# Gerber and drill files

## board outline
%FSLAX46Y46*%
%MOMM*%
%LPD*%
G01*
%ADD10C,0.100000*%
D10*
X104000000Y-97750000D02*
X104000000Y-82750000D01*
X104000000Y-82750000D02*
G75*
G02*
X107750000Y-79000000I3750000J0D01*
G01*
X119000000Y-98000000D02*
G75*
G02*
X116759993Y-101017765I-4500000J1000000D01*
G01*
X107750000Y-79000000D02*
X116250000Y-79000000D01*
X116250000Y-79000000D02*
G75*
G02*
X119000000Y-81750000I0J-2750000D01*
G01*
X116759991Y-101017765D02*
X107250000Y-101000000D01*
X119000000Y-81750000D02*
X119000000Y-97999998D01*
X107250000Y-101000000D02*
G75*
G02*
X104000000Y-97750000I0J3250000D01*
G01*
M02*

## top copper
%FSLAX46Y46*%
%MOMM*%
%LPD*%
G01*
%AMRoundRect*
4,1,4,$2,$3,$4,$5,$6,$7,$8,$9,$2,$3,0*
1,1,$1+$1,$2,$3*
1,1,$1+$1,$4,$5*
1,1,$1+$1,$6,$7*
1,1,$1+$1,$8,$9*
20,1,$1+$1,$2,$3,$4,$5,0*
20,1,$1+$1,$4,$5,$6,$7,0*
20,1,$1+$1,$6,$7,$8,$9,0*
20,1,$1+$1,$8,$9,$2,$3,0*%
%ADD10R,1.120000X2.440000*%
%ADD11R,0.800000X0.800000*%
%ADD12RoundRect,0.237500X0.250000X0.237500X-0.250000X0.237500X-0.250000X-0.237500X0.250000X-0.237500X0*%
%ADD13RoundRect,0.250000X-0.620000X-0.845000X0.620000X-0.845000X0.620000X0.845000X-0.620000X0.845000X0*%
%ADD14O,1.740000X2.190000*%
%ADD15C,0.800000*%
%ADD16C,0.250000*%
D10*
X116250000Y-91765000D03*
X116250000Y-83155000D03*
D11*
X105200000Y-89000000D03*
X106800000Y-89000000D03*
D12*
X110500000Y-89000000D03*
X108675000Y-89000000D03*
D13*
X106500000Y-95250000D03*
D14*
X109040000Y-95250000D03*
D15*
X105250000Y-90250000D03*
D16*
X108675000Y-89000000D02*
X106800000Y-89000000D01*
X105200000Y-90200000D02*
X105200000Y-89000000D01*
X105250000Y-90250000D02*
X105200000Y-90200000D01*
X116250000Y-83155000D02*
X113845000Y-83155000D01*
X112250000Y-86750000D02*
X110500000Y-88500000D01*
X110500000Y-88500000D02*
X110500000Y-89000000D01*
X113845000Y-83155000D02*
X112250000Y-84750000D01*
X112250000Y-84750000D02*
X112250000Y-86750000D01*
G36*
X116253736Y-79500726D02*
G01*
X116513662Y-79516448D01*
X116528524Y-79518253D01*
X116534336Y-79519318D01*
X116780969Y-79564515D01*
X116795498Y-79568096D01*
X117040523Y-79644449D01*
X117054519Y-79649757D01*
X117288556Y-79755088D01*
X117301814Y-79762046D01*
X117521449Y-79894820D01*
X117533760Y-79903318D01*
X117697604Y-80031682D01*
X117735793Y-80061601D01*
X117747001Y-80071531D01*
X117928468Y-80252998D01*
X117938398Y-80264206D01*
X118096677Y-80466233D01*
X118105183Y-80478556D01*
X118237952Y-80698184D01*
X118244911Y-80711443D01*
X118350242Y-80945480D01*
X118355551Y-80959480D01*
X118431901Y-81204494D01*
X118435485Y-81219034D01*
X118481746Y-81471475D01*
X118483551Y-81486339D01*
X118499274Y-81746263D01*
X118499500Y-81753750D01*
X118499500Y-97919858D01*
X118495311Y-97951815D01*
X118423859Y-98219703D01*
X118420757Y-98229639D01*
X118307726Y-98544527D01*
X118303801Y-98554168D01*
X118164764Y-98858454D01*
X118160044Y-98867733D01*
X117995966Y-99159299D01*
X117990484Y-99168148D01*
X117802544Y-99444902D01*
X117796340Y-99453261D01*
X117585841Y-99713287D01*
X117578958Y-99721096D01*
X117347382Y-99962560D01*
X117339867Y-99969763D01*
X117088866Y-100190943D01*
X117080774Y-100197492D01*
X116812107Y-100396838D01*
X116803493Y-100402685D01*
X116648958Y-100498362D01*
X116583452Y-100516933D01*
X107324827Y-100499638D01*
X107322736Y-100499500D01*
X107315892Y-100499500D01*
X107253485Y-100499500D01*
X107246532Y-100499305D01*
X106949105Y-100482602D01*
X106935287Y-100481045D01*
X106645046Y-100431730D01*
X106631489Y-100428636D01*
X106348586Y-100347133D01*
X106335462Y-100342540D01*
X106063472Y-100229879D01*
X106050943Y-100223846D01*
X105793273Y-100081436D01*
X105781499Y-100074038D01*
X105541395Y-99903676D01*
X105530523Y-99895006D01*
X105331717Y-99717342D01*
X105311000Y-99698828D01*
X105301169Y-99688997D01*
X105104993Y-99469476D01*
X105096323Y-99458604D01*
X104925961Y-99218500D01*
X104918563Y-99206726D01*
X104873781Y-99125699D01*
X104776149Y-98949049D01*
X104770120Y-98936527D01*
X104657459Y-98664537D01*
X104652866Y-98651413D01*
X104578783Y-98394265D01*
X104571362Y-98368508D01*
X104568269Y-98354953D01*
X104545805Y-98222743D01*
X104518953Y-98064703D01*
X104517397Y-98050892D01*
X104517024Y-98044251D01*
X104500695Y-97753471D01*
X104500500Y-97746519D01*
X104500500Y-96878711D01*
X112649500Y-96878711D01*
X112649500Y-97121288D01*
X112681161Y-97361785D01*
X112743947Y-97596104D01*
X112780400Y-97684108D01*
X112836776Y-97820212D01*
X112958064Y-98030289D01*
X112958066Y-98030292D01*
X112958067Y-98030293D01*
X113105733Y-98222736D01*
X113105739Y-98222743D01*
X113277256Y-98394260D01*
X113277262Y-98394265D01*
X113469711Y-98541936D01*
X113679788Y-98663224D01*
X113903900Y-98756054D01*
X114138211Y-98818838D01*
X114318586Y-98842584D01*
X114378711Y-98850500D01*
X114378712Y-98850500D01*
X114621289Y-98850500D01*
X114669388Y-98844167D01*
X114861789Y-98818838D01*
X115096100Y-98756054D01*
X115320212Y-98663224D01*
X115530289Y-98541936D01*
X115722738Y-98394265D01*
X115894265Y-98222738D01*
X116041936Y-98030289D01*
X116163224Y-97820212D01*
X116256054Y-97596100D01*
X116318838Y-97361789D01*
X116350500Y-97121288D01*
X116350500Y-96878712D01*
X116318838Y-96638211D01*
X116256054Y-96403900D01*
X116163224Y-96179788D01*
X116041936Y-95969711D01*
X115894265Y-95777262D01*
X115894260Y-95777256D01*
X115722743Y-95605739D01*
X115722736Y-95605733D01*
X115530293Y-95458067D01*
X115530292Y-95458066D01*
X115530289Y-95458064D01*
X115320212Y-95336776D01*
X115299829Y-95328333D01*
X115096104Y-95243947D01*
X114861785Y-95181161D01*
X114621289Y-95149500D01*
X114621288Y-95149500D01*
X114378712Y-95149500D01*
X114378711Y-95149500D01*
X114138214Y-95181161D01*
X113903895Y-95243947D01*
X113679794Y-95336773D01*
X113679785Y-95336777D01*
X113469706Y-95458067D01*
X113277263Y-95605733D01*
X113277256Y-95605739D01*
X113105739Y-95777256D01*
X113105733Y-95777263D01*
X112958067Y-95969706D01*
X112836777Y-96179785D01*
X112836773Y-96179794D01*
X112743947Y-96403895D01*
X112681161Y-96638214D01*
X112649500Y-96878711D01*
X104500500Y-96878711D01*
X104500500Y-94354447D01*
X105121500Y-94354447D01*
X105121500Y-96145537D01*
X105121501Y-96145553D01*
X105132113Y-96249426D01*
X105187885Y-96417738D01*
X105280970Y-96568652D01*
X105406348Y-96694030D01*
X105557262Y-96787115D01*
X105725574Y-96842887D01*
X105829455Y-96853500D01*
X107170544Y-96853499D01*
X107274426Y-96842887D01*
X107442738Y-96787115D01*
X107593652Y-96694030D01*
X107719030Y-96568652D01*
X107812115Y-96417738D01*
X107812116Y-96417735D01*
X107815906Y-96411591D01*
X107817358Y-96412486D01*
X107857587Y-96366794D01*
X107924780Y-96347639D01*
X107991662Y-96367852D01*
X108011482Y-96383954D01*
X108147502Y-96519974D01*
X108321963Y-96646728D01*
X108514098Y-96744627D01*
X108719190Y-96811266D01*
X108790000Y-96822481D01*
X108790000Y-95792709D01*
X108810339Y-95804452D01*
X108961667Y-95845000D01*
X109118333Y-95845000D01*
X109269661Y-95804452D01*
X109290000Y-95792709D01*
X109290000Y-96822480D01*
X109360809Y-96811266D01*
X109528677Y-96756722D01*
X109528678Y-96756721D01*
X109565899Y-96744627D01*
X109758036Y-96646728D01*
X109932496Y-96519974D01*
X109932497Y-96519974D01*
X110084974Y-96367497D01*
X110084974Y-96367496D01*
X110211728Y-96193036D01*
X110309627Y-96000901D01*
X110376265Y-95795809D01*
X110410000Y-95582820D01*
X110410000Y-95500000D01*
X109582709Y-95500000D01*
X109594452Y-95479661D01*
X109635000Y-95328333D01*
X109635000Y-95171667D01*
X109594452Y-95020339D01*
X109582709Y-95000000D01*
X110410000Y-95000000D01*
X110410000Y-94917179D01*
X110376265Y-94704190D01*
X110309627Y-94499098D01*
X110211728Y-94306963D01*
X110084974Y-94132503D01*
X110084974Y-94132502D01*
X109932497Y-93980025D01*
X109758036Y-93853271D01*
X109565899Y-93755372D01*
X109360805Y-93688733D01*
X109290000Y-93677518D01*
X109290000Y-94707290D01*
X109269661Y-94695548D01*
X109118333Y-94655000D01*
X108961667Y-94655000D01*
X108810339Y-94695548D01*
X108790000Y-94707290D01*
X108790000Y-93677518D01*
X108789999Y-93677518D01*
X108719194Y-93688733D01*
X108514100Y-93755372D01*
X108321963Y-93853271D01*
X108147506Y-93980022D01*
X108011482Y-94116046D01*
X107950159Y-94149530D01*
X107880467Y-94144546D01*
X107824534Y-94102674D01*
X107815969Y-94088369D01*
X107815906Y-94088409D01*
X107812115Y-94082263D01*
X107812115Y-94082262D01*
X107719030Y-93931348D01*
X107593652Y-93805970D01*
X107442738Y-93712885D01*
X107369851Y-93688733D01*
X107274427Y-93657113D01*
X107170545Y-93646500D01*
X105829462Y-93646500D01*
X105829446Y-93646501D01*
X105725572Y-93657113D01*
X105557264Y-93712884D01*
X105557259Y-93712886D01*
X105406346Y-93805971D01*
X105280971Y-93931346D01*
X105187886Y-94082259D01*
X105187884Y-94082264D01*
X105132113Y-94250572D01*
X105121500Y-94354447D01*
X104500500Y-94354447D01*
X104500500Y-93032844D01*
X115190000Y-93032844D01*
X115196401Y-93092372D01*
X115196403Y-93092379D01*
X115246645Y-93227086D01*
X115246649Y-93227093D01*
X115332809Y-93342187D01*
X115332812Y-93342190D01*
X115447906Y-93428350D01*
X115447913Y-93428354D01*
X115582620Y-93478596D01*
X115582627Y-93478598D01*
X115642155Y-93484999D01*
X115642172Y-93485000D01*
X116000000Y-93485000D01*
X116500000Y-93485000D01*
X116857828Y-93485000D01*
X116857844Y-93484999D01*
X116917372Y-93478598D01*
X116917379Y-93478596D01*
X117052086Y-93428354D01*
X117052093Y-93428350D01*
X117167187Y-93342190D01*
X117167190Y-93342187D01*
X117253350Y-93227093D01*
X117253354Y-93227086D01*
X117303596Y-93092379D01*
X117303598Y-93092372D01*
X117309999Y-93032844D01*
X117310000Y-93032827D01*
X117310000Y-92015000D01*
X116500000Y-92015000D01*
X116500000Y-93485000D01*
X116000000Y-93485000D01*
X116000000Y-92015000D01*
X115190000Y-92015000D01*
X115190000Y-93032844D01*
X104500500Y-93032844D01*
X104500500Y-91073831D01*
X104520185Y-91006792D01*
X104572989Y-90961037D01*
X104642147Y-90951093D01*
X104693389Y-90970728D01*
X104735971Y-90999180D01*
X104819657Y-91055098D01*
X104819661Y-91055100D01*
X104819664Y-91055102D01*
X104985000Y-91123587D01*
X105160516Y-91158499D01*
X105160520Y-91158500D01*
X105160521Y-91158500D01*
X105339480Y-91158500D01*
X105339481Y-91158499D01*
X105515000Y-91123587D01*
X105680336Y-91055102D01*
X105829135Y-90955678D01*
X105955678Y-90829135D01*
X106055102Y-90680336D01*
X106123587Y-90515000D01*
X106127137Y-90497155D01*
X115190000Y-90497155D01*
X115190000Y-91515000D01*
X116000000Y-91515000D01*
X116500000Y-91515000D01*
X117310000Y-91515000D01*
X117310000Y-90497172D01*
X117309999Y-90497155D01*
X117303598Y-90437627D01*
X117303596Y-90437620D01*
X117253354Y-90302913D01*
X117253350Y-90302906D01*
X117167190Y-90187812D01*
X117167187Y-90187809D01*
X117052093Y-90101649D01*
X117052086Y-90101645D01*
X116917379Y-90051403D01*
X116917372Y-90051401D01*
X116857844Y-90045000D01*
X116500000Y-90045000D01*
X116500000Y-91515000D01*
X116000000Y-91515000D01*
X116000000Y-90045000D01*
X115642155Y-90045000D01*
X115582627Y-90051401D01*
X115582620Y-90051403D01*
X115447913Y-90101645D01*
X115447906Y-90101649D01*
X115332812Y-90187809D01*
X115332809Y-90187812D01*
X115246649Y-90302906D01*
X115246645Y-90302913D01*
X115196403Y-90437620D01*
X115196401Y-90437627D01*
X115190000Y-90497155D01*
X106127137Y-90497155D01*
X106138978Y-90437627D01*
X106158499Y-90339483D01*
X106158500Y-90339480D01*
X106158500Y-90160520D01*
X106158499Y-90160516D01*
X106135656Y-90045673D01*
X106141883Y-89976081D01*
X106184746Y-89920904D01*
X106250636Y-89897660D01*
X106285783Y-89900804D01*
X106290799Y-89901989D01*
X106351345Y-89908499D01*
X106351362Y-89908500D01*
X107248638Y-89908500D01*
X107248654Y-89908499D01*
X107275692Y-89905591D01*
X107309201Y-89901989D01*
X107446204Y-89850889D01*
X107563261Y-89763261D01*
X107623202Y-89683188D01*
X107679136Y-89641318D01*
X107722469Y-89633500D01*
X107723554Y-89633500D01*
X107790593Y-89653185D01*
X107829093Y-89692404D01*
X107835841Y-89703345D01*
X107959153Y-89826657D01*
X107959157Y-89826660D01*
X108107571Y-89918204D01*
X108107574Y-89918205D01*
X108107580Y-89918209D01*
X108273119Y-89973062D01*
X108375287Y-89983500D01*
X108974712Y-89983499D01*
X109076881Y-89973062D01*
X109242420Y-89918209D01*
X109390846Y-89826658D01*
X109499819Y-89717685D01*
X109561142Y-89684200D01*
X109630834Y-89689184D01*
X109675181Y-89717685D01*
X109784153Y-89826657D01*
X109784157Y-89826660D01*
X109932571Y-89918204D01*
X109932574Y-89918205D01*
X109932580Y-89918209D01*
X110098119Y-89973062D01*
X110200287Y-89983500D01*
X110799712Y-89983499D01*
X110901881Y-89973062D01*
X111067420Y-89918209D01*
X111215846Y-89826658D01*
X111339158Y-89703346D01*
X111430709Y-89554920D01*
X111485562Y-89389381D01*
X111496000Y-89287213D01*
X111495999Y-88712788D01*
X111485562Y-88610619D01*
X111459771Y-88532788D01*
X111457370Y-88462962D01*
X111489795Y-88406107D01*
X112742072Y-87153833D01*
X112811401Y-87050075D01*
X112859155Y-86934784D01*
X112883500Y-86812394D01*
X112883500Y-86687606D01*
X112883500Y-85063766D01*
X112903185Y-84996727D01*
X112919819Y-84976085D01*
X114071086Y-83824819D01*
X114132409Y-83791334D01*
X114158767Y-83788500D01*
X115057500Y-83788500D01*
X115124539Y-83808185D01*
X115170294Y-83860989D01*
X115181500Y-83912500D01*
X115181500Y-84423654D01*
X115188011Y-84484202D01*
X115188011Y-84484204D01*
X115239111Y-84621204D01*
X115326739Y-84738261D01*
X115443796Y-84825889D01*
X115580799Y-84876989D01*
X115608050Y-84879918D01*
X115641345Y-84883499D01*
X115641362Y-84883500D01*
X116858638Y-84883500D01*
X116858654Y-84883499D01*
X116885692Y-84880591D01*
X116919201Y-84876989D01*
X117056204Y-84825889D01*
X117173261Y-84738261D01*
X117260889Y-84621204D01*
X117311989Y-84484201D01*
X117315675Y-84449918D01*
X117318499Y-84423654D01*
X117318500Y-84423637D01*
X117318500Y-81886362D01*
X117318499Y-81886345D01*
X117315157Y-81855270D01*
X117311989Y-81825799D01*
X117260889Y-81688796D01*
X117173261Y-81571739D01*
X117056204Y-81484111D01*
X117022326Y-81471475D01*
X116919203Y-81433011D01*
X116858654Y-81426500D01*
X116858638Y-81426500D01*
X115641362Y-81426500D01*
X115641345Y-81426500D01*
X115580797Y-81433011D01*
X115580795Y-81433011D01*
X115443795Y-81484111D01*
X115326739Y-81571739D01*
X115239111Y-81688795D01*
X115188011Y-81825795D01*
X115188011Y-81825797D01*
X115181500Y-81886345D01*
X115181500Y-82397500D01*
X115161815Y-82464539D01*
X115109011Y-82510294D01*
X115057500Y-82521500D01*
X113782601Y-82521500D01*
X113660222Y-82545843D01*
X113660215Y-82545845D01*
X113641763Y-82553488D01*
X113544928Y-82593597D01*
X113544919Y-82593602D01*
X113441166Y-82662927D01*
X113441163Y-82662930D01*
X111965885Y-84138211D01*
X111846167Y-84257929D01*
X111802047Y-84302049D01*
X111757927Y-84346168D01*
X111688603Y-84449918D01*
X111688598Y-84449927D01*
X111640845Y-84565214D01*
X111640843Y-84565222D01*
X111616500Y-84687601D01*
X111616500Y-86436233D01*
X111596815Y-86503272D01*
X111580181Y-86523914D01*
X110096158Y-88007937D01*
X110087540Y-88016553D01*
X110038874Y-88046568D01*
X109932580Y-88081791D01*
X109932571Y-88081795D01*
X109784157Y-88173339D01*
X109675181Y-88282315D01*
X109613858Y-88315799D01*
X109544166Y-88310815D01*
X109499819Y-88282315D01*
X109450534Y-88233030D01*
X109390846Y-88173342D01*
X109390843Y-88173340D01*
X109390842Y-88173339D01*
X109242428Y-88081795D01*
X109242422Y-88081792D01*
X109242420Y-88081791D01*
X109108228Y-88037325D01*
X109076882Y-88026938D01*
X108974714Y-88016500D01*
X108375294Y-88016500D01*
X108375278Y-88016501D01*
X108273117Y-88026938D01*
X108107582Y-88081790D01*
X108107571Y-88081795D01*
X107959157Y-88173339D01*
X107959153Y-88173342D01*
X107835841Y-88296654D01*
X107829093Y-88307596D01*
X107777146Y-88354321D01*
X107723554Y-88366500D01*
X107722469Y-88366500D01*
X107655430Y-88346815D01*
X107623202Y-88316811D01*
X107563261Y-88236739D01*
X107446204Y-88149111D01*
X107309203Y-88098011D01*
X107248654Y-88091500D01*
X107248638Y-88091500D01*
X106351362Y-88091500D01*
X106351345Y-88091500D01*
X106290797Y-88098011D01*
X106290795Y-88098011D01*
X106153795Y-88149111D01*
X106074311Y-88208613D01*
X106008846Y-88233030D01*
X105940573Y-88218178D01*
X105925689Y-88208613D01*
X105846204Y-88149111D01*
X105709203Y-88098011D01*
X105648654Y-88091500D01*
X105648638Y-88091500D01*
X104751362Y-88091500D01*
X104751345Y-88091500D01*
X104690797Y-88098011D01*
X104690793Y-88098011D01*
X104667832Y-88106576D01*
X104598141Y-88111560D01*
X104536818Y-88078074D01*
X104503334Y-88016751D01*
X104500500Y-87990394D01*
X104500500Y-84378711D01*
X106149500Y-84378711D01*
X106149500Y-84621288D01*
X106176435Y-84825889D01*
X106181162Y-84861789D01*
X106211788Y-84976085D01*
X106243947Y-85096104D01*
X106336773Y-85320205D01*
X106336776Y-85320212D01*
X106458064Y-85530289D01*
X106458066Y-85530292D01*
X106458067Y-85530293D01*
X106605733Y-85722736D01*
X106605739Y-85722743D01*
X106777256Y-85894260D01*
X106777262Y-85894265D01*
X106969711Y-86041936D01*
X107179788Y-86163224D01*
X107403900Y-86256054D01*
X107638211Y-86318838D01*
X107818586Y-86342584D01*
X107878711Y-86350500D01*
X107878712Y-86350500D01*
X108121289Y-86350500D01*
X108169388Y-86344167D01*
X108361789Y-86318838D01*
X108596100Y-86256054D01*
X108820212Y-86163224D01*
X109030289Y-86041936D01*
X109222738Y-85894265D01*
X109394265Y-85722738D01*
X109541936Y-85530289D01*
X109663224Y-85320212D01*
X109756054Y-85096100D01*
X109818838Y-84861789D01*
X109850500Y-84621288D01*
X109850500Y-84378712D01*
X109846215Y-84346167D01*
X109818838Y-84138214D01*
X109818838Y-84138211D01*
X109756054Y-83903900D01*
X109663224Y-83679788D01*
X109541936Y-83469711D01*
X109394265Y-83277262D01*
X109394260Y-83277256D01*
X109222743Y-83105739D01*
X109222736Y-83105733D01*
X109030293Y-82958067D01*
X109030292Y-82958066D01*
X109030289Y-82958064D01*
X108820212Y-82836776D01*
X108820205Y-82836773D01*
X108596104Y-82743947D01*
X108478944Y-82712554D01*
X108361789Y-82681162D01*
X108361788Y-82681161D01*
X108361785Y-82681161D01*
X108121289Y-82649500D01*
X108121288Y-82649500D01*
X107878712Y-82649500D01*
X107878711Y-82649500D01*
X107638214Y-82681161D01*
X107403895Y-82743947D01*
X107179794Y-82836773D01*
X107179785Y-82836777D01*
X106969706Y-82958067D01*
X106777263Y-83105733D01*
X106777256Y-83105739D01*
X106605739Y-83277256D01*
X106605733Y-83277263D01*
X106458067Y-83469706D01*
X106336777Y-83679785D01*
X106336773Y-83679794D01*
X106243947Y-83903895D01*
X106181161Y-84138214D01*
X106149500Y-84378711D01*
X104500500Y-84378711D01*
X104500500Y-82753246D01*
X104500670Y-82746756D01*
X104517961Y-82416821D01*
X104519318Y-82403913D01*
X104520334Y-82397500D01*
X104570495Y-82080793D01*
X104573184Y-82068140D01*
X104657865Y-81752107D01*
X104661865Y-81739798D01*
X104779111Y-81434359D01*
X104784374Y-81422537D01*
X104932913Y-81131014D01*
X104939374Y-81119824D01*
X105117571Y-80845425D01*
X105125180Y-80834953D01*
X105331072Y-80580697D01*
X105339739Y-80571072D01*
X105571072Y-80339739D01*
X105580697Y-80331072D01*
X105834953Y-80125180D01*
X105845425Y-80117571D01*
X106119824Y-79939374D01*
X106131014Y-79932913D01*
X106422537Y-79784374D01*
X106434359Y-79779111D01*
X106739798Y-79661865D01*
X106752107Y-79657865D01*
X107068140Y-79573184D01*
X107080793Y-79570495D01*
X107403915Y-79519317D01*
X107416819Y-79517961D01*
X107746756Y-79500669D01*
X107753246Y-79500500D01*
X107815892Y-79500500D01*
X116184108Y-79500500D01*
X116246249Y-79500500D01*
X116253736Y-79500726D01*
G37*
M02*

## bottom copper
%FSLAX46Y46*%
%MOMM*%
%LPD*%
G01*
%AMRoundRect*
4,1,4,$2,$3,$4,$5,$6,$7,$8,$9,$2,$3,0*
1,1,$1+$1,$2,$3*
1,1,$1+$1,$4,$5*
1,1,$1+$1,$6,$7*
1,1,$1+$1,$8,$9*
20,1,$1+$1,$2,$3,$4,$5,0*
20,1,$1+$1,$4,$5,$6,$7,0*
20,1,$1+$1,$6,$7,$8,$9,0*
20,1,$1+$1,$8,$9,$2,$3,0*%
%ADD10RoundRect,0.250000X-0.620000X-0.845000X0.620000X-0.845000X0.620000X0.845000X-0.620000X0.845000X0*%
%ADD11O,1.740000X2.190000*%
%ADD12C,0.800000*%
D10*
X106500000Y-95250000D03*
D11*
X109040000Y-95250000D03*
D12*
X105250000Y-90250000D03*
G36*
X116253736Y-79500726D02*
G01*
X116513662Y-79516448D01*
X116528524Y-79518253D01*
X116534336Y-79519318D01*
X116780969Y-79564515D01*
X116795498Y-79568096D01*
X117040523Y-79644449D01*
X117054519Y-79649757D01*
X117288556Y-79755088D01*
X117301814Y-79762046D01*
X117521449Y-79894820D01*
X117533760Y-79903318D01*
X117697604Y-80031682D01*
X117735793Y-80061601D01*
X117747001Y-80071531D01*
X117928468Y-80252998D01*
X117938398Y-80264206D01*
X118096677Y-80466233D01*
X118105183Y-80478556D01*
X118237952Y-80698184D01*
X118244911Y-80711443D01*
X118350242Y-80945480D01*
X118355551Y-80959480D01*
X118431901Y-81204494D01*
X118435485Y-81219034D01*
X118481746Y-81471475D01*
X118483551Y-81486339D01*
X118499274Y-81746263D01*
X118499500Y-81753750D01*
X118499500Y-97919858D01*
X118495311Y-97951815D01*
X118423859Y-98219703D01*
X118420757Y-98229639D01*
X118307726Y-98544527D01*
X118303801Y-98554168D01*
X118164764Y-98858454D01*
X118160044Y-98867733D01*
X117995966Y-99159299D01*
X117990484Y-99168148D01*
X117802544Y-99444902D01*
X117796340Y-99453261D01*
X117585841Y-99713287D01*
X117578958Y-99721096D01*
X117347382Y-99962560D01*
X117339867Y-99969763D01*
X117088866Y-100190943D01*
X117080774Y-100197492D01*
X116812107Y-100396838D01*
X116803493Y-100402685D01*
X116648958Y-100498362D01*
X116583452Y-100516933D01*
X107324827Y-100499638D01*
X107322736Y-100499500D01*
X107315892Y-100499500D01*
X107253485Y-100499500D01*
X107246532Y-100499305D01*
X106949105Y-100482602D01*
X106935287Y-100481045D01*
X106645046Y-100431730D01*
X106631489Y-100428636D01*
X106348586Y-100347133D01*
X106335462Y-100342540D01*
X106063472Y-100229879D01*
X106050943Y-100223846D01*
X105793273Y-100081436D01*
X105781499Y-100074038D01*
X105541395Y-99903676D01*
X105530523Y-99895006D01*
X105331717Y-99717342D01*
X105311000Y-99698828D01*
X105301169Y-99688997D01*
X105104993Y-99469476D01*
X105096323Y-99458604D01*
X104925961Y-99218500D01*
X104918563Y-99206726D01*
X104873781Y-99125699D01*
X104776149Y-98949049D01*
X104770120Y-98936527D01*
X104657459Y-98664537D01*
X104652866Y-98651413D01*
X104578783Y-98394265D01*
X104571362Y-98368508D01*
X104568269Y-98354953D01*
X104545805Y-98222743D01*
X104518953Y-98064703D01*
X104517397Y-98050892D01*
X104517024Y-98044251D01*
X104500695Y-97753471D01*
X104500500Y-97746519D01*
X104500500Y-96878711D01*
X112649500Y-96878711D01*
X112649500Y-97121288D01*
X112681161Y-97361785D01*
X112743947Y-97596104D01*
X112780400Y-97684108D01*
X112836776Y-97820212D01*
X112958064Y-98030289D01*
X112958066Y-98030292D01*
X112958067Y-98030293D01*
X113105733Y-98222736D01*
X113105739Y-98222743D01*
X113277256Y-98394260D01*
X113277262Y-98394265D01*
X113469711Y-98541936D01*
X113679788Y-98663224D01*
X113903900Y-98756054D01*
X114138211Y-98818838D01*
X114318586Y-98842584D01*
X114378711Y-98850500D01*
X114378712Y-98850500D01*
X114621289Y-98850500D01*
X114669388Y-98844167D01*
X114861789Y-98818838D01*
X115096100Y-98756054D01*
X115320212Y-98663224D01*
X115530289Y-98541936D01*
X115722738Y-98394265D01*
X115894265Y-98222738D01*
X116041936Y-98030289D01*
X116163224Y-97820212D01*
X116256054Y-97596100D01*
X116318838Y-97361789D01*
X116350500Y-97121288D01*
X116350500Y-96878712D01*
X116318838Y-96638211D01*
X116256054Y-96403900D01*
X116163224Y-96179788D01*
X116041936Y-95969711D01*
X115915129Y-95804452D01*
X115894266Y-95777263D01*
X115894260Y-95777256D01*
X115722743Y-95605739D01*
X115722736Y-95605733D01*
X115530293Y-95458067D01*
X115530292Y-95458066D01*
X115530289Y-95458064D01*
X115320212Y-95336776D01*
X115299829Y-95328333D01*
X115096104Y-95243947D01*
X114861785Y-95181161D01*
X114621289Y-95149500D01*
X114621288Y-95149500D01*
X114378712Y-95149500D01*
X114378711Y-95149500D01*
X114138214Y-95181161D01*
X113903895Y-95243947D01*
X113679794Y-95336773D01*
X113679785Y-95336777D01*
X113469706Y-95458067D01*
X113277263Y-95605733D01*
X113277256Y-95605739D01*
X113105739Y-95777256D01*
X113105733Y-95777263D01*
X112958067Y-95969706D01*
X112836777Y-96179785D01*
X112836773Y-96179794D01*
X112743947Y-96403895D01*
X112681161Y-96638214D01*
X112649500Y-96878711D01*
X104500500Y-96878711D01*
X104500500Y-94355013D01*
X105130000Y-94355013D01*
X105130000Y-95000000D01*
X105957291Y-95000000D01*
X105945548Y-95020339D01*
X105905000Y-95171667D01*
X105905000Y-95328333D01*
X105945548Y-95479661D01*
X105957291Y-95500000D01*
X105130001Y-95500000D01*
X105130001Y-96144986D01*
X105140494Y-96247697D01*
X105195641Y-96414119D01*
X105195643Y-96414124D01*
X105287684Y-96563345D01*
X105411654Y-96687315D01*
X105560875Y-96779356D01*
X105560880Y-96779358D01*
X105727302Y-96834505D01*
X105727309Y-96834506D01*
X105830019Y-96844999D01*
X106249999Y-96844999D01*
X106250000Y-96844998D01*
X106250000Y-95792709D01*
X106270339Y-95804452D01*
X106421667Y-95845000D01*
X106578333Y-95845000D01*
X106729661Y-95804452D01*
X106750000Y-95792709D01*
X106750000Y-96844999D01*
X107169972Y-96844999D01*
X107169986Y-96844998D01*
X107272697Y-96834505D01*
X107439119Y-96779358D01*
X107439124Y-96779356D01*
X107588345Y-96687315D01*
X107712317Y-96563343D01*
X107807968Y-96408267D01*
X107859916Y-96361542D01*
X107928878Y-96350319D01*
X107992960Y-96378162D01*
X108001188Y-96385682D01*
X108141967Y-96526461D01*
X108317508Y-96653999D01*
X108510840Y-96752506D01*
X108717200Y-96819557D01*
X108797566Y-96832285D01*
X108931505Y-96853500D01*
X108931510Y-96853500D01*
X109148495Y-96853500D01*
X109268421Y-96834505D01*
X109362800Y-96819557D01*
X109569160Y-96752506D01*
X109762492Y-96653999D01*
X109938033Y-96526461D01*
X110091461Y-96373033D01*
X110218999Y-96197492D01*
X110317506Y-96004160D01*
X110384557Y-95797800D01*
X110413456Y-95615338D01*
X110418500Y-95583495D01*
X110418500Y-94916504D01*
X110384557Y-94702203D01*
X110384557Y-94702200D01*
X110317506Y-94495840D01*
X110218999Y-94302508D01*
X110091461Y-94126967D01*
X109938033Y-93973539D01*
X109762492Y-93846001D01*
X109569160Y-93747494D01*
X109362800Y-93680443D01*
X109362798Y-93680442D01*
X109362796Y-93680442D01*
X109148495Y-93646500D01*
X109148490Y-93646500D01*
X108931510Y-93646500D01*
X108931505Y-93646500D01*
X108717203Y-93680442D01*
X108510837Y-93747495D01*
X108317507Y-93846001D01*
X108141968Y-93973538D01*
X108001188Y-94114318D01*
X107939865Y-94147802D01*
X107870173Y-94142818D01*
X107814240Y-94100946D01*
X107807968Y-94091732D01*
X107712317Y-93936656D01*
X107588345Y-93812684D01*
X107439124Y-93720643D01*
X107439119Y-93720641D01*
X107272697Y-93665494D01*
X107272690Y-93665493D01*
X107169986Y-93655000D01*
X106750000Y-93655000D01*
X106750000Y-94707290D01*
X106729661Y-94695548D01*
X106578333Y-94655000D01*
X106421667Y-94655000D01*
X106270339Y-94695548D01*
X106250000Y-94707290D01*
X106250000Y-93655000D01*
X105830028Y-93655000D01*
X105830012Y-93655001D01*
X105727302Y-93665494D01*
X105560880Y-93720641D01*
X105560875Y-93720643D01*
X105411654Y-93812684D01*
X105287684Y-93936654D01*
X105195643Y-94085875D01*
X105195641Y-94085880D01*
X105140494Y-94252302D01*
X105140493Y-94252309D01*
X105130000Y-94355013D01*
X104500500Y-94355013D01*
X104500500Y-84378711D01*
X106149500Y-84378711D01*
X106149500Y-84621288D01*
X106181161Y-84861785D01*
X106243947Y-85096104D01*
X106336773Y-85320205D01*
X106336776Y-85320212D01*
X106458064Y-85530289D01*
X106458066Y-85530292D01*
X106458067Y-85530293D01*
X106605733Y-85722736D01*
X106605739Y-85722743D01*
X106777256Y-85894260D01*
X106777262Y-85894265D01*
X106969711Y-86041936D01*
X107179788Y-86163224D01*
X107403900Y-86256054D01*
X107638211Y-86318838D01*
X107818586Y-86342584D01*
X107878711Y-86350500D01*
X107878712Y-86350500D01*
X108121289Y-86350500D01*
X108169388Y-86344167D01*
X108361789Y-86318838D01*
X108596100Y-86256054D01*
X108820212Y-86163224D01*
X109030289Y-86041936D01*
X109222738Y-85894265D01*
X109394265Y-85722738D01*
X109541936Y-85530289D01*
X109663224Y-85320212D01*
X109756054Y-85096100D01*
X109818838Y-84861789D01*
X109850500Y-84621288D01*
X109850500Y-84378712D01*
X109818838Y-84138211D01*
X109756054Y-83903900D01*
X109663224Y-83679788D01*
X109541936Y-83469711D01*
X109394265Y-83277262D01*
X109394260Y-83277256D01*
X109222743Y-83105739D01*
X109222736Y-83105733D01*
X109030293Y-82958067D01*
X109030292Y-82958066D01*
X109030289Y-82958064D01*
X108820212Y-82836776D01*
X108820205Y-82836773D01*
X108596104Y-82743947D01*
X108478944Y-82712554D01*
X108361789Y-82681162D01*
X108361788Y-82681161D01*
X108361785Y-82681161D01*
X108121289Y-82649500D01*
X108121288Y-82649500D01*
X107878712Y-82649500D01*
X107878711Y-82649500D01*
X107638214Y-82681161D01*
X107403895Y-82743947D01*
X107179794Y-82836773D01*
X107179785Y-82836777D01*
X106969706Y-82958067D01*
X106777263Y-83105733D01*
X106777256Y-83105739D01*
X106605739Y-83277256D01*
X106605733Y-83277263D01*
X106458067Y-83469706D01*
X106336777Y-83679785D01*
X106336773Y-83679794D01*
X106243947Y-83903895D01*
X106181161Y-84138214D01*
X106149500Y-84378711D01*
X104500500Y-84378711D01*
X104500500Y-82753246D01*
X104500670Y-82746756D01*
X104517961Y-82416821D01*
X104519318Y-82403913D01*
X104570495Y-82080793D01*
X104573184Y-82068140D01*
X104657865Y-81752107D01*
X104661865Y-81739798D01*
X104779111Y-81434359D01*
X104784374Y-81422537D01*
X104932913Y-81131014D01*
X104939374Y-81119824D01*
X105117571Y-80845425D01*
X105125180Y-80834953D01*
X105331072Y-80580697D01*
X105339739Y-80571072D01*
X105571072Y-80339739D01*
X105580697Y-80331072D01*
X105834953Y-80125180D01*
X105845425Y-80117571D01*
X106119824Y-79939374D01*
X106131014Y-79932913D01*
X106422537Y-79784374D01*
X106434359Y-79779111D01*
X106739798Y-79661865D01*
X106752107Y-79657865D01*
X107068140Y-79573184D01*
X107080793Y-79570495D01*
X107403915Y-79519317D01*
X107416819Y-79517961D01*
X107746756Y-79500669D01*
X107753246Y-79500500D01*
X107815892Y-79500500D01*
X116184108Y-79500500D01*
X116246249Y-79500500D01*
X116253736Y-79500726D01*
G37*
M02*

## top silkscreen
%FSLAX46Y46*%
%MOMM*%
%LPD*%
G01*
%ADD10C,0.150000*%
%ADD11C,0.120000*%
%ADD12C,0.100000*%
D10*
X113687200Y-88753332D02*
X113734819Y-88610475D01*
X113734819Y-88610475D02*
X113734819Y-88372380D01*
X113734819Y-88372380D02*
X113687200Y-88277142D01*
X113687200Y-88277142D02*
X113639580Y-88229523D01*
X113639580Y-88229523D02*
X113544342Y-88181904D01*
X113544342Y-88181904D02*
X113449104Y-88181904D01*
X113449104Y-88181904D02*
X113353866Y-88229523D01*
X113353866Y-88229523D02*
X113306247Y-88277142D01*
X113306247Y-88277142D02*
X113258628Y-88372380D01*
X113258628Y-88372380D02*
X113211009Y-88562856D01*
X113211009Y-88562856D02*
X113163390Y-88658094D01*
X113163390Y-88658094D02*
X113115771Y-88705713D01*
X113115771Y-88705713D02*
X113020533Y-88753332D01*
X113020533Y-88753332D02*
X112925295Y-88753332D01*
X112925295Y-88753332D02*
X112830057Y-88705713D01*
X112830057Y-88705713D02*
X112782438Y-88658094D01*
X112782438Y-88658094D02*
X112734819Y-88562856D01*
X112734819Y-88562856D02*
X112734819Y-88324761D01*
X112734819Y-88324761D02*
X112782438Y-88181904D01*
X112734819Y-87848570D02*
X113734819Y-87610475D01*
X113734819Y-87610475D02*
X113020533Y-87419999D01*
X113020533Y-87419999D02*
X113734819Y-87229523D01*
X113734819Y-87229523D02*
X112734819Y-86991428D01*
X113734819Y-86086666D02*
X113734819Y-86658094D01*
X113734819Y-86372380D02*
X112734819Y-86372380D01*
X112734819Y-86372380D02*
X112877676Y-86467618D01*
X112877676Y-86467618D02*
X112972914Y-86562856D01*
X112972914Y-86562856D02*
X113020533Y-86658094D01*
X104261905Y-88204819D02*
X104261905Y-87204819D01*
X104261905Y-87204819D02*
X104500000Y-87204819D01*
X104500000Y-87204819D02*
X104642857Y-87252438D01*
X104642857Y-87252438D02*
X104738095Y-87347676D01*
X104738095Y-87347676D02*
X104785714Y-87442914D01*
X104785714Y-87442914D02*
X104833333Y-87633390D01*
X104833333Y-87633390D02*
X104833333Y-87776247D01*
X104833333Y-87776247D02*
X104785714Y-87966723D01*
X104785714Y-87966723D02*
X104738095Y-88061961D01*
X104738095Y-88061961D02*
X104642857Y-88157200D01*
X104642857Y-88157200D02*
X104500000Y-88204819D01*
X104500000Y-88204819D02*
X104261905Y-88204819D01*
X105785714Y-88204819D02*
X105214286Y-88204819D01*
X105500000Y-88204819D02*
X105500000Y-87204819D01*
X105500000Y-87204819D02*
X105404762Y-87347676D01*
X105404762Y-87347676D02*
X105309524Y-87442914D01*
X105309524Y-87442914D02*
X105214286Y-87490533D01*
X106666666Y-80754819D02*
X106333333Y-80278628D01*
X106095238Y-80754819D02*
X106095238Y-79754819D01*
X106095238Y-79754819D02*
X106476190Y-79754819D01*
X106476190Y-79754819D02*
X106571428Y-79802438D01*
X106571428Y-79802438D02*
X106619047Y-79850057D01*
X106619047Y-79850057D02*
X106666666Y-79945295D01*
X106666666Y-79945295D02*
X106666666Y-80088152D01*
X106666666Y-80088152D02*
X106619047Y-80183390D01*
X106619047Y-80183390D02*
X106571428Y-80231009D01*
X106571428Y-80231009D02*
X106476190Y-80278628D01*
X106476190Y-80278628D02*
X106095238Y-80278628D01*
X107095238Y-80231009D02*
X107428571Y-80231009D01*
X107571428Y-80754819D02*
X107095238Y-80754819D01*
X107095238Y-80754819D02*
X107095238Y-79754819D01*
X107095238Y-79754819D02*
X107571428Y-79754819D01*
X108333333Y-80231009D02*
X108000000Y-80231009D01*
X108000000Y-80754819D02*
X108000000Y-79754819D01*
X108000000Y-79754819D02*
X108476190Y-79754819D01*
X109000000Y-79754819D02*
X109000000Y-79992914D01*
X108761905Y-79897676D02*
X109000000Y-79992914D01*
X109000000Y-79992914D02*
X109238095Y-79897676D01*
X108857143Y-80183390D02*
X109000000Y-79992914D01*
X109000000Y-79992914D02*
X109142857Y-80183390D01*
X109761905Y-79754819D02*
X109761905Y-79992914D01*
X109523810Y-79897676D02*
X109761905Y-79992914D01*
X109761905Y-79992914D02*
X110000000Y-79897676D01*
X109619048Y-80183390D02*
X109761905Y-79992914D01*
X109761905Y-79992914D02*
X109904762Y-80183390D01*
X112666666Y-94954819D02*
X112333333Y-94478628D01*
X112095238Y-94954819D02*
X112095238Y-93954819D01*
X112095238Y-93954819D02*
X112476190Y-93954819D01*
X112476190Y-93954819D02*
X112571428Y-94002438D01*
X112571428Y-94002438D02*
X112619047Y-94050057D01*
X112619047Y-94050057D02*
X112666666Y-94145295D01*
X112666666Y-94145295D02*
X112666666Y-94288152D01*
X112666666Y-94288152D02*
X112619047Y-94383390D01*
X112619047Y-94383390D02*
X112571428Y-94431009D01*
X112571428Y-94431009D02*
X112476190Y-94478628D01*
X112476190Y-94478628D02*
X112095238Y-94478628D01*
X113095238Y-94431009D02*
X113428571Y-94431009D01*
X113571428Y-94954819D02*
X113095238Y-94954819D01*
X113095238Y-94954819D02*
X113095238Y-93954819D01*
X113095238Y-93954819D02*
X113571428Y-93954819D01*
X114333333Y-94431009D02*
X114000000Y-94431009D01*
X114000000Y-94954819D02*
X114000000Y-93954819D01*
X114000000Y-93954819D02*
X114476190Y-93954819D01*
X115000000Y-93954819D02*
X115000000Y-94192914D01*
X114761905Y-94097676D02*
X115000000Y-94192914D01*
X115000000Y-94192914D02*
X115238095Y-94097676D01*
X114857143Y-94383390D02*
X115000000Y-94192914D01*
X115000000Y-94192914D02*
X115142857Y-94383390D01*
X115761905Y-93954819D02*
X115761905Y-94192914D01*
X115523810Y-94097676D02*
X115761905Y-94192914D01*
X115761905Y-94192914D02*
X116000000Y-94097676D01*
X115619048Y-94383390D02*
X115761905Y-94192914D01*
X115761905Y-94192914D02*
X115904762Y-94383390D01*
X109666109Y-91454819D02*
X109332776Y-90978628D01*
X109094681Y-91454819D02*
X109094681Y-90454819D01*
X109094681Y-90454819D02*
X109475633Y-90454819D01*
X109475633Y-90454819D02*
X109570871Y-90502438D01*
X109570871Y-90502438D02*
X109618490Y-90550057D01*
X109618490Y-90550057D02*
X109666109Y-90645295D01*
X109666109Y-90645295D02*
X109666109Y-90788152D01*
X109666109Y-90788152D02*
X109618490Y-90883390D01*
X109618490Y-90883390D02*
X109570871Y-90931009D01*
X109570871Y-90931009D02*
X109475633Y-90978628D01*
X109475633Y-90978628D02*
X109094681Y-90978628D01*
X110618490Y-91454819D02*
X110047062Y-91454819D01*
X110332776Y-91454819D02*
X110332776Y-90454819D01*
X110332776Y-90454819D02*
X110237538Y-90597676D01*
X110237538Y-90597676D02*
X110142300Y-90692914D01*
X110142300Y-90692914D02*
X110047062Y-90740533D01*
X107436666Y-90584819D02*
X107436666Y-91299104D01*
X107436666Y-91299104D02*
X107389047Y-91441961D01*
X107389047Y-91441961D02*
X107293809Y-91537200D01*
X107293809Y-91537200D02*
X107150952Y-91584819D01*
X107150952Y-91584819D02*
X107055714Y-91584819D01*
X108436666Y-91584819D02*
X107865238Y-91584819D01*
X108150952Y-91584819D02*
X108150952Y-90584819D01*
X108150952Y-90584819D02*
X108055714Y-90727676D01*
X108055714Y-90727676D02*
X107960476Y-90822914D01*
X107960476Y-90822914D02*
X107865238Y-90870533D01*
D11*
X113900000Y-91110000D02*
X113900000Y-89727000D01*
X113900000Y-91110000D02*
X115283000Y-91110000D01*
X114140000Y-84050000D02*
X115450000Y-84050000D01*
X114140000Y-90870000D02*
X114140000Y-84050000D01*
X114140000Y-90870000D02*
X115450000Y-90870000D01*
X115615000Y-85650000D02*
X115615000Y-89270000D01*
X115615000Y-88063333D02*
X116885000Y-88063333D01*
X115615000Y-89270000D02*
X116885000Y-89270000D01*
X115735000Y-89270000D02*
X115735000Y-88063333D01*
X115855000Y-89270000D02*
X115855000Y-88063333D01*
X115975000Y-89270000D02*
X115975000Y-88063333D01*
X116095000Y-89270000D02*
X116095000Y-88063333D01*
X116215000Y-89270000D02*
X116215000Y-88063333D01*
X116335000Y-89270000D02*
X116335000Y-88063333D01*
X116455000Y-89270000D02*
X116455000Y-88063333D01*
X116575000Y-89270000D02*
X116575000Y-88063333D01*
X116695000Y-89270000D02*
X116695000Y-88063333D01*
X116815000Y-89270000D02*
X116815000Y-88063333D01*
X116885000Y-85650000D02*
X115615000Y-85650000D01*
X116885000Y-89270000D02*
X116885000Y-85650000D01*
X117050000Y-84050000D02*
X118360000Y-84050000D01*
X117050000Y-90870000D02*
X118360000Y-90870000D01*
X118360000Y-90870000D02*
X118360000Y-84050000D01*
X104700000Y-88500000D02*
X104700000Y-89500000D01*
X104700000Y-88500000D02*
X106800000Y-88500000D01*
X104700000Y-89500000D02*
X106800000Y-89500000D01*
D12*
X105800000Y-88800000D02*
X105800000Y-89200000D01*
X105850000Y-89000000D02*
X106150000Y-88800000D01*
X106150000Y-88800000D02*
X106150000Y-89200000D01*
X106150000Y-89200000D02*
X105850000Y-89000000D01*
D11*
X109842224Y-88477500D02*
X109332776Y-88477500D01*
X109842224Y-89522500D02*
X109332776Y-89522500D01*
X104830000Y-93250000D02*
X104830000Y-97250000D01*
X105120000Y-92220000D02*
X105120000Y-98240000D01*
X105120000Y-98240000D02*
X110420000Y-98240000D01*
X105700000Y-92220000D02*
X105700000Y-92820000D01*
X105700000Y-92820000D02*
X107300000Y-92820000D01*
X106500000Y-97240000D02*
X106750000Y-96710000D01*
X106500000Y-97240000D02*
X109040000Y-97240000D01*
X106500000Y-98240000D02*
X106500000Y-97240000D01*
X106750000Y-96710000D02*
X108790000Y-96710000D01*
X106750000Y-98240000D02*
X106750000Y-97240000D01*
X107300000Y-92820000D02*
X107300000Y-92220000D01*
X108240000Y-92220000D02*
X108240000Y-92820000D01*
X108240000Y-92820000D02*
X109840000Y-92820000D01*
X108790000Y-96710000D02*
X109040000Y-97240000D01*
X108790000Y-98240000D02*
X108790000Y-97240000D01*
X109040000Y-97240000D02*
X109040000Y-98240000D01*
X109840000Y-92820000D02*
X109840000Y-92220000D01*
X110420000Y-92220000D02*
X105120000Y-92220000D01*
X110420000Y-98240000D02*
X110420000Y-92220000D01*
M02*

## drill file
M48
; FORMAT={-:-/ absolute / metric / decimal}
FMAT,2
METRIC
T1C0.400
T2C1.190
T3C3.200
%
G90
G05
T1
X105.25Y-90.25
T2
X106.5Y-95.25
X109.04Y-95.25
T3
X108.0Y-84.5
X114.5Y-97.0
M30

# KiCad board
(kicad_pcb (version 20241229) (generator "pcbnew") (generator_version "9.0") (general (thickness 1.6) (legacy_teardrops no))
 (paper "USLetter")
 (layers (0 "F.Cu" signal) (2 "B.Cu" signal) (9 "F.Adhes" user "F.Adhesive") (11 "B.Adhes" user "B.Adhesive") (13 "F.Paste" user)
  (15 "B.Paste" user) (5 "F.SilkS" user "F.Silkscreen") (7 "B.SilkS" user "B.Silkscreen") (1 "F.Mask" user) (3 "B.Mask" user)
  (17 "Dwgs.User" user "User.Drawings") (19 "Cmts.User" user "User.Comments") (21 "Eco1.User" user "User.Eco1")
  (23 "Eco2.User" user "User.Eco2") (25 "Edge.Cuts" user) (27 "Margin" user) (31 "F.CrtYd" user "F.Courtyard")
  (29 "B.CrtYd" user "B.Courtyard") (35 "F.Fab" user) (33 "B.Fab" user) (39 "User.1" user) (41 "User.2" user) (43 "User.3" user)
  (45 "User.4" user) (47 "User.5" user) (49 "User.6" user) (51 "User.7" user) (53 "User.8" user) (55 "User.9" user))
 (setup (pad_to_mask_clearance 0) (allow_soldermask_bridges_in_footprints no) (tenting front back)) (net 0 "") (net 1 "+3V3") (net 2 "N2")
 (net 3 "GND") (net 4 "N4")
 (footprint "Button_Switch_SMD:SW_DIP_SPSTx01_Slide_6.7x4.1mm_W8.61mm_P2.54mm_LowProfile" (layer "F.Cu") (at 116.25 87.46 90)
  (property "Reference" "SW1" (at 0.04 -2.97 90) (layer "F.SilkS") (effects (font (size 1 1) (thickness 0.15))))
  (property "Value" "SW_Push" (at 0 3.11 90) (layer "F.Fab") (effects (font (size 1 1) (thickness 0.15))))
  (fp_line (start -3.65 -2.35) (end -2.267 -2.35) (stroke (width 0.12) (type solid)) (layer "F.SilkS"))
  (fp_line (start -3.65 -2.35) (end -3.65 -0.967) (stroke (width 0.12) (type solid)) (layer "F.SilkS"))
  (fp_line (start 3.41 -2.11) (end 3.41 -0.8) (stroke (width 0.12) (type solid)) (layer "F.SilkS"))
  (fp_line (start -3.41 -2.11) (end 3.41 -2.11) (stroke (width 0.12) (type solid)) (layer "F.SilkS"))
  (fp_line (start -3.41 -2.11) (end -3.41 -0.8) (stroke (width 0.12) (type solid)) (layer "F.SilkS"))
  (fp_line (start 1.81 -0.635) (end -1.81 -0.635) (stroke (width 0.12) (type solid)) (layer "F.SilkS"))
  (fp_line (start -0.603333 -0.635) (end -0.603333 0.635) (stroke (width 0.12) (type solid)) (layer "F.SilkS"))
  (fp_line (start -1.81 -0.635) (end -1.81 0.635) (stroke (width 0.12) (type solid)) (layer "F.SilkS"))
  (fp_line (start -1.81 -0.515) (end -0.603333 -0.515) (stroke (width 0.12) (type solid)) (layer "F.SilkS"))
  (fp_line (start -1.81 -0.395) (end -0.603333 -0.395) (stroke (width 0.12) (type solid)) (layer "F.SilkS"))
  (fp_line (start -1.81 -0.275) (end -0.603333 -0.275) (stroke (width 0.12) (type solid)) (layer "F.SilkS"))
  (fp_line (start -1.81 -0.155) (end -0.603333 -0.155) (stroke (width 0.12) (type solid)) (layer "F.SilkS"))
  (fp_line (start -1.81 -0.035) (end -0.603333 -0.035) (stroke (width 0.12) (type solid)) (layer "F.SilkS"))
  (fp_line (start -1.81 0.085) (end -0.603333 0.085) (stroke (width 0.12) (type solid)) (layer "F.SilkS"))
  (fp_line (start -1.81 0.205) (end -0.603333 0.205) (stroke (width 0.12) (type solid)) (layer "F.SilkS"))
  (fp_line (start -1.81 0.325) (end -0.603333 0.325) (stroke (width 0.12) (type solid)) (layer "F.SilkS"))
  (fp_line (start -1.81 0.445) (end -0.603333 0.445) (stroke (width 0.12) (type solid)) (layer "F.SilkS"))
  (fp_line (start -1.81 0.565) (end -0.603333 0.565) (stroke (width 0.12) (type solid)) (layer "F.SilkS"))
  (fp_line (start 1.81 0.635) (end 1.81 -0.635) (stroke (width 0.12) (type solid)) (layer "F.SilkS"))
  (fp_line (start -1.81 0.635) (end 1.81 0.635) (stroke (width 0.12) (type solid)) (layer "F.SilkS"))
  (fp_line (start 3.41 0.8) (end 3.41 2.11) (stroke (width 0.12) (type solid)) (layer "F.SilkS"))
  (fp_line (start -3.41 0.8) (end -3.41 2.11) (stroke (width 0.12) (type solid)) (layer "F.SilkS"))
  (fp_line (start -3.41 2.11) (end 3.41 2.11) (stroke (width 0.12) (type solid)) (layer "F.SilkS"))
  (pad "1" smd rect (at -4.305 0 90) (size 2.44 1.12) (layers "F.Cu" "F.Mask" "F.Paste") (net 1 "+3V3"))
  (pad "2" smd rect (at 4.305 0 90) (size 2.44 1.12) (layers "F.Cu" "F.Mask" "F.Paste") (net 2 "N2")))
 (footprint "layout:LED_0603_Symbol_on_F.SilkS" (layer "F.Cu") (at 106 89)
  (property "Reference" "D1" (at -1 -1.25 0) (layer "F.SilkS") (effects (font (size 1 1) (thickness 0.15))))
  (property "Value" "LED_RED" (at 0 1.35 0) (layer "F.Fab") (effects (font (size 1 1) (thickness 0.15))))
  (fp_line (start -1.3 -0.5) (end -1.3 0.5) (stroke (width 0.12) (type solid)) (layer "F.SilkS"))
  (fp_line (start -1.3 -0.5) (end 0.8 -0.5) (stroke (width 0.12) (type solid)) (layer "F.SilkS"))
  (fp_line (start -1.3 0.5) (end 0.8 0.5) (stroke (width 0.12) (type solid)) (layer "F.SilkS"))
  (fp_line (start -0.2 -0.2) (end -0.2 0.2) (stroke (width 0.1) (type solid)) (layer "F.SilkS"))
  (fp_line (start -0.15 0) (end 0.15 -0.2) (stroke (width 0.1) (type solid)) (layer "F.SilkS"))
  (fp_line (start 0.15 -0.2) (end 0.15 0.2) (stroke (width 0.1) (type solid)) (layer "F.SilkS"))
  (fp_line (start 0.15 0.2) (end -0.15 0) (stroke (width 0.1) (type solid)) (layer "F.SilkS"))
  (pad "1" smd rect (at -0.8 0 180) (size 0.8 0.8) (layers "F.Cu" "F.Mask" "F.Paste") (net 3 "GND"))
  (pad "2" smd rect (at 0.8 0 180) (size 0.8 0.8) (layers "F.Cu" "F.Mask" "F.Paste") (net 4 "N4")))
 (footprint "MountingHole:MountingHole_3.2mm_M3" (layer "F.Cu") (at 108 84.5)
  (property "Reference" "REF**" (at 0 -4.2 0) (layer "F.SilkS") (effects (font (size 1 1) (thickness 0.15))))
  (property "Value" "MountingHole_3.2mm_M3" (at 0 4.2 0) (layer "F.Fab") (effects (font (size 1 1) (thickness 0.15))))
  (pad "" np_thru_hole circle (at 0 0) (size 3.2 3.2) (drill 3.2) (layers "*.Cu" "*.Mask")))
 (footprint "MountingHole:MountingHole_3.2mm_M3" (layer "F.Cu") (at 114.5 97)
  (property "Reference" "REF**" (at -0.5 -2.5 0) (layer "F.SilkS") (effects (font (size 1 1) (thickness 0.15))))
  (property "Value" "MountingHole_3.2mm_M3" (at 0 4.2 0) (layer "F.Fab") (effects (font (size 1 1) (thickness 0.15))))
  (pad "" np_thru_hole circle (at 0 0) (size 3.2 3.2) (drill 3.2) (layers "*.Cu" "*.Mask")))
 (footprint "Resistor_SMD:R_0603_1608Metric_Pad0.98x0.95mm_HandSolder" (layer "F.Cu") (at 109.5875 89 180)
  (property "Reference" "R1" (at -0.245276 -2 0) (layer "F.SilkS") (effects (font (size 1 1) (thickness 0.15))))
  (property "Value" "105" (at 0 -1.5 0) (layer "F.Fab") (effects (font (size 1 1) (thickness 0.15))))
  (fp_line (start -0.254724 0.5225) (end 0.254724 0.5225) (stroke (width 0.12) (type solid)) (layer "F.SilkS"))
  (fp_line (start -0.254724 -0.5225) (end 0.254724 -0.5225) (stroke (width 0.12) (type solid)) (layer "F.SilkS"))
  (pad "1" smd roundrect (at -0.9125 0 180) (size 0.975 0.95) (layers "F.Cu" "F.Mask" "F.Paste") (roundrect_rratio 0.25) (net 2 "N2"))
  (pad "2" smd roundrect (at 0.9125 0 180) (size 0.975 0.95) (layers "F.Cu" "F.Mask" "F.Paste") (roundrect_rratio 0.25) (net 4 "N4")))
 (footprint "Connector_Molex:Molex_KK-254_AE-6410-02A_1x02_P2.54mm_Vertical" (layer "F.Cu") (at 106.5 95.25)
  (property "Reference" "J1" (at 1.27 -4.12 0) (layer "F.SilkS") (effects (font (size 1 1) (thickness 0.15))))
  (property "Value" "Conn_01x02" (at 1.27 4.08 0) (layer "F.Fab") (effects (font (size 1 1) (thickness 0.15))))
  (fp_line (start -1.67 -2) (end -1.67 2) (stroke (width 0.12) (type solid)) (layer "F.SilkS"))
  (fp_line (start -1.38 -3.03) (end -1.38 2.99) (stroke (width 0.12) (type solid)) (layer "F.SilkS"))
  (fp_line (start -1.38 2.99) (end 3.92 2.99) (stroke (width 0.12) (type solid)) (layer "F.SilkS"))
  (fp_line (start -0.8 -3.03) (end -0.8 -2.43) (stroke (width 0.12) (type solid)) (layer "F.SilkS"))
  (fp_line (start -0.8 -2.43) (end 0.8 -2.43) (stroke (width 0.12) (type solid)) (layer "F.SilkS"))
  (fp_line (start 0 1.99) (end 0.25 1.46) (stroke (width 0.12) (type solid)) (layer "F.SilkS"))
  (fp_line (start 0 1.99) (end 2.54 1.99) (stroke (width 0.12) (type solid)) (layer "F.SilkS"))
  (fp_line (start 0 2.99) (end 0 1.99) (stroke (width 0.12) (type solid)) (layer "F.SilkS"))
  (fp_line (start 0.25 1.46) (end 2.29 1.46) (stroke (width 0.12) (type solid)) (layer "F.SilkS"))
  (fp_line (start 0.25 2.99) (end 0.25 1.99) (stroke (width 0.12) (type solid)) (layer "F.SilkS"))
  (fp_line (start 0.8 -2.43) (end 0.8 -3.03) (stroke (width 0.12) (type solid)) (layer "F.SilkS"))
  (fp_line (start 1.74 -3.03) (end 1.74 -2.43) (stroke (width 0.12) (type solid)) (layer "F.SilkS"))
  (fp_line (start 1.74 -2.43) (end 3.34 -2.43) (stroke (width 0.12) (type solid)) (layer "F.SilkS"))
  (fp_line (start 2.29 1.46) (end 2.54 1.99) (stroke (width 0.12) (type solid)) (layer "F.SilkS"))
  (fp_line (start 2.29 2.99) (end 2.29 1.99) (stroke (width 0.12) (type solid)) (layer "F.SilkS"))
  (fp_line (start 2.54 1.99) (end 2.54 2.99) (stroke (width 0.12) (type solid)) (layer "F.SilkS"))
  (fp_line (start 3.34 -2.43) (end 3.34 -3.03) (stroke (width 0.12) (type solid)) (layer "F.SilkS"))
  (fp_line (start 3.92 -3.03) (end -1.38 -3.03) (stroke (width 0.12) (type solid)) (layer "F.SilkS"))
  (fp_line (start 3.92 2.99) (end 3.92 -3.03) (stroke (width 0.12) (type solid)) (layer "F.SilkS"))
  (pad "1" thru_hole roundrect (at 0 0) (size 1.74 2.19) (drill 1.19) (layers "*.Cu" "*.Mask") (remove_unused_layers no)
   (roundrect_rratio 0.143678) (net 3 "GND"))
  (pad "2" thru_hole oval (at 2.54 0) (size 1.74 2.19) (drill 1.19) (layers "*.Cu" "*.Mask") (remove_unused_layers no) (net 1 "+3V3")))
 (gr_line (start 104 97.75) (end 104 82.75) (stroke (width 0.1) (type default)) (layer "Edge.Cuts"))
 (gr_arc (start 104 82.75) (mid 105.09835 80.09835) (end 107.75 79) (stroke (width 0.1) (type default)) (layer "Edge.Cuts"))
 (gr_arc (start 119 98) (mid 118.2015 99.747526) (end 116.759993 101.017765) (stroke (width 0.1) (type default)) (layer "Edge.Cuts"))
 (gr_line (start 107.75 79) (end 116.25 79) (stroke (width 0.1) (type default)) (layer "Edge.Cuts"))
 (gr_arc (start 116.25 79) (mid 118.194544 79.805456) (end 119 81.75) (stroke (width 0.1) (type default)) (layer "Edge.Cuts"))
 (gr_line (start 116.759991 101.017765) (end 107.25 101) (stroke (width 0.1) (type default)) (layer "Edge.Cuts"))
 (gr_line (start 119 81.75) (end 119 97.999998) (stroke (width 0.1) (type default)) (layer "Edge.Cuts"))
 (gr_arc (start 107.25 101) (mid 104.951903 100.048097) (end 104 97.75) (stroke (width 0.1) (type default)) (layer "Edge.Cuts"))
 (segment (start 108.675 89) (end 106.8 89) (width 0.25) (layer "F.Cu") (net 4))
 (segment (start 105.2 90.2) (end 105.2 89) (width 0.25) (layer "F.Cu") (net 3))
 (segment (start 105.25 90.25) (end 105.2 90.2) (width 0.25) (layer "F.Cu") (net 3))
 (via (at 105.25 90.25) (size 0.8) (drill 0.4) (layers "F.Cu" "B.Cu") (free yes) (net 3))
 (segment (start 116.25 83.155) (end 113.845 83.155) (width 0.25) (layer "F.Cu") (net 2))
 (segment (start 112.25 86.75) (end 110.5 88.5) (width 0.25) (layer "F.Cu") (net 2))
 (segment (start 110.5 88.5) (end 110.5 89) (width 0.25) (layer "F.Cu") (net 2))
 (segment (start 113.845 83.155) (end 112.25 84.75) (width 0.25) (layer "F.Cu") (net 2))
 (segment (start 112.25 84.75) (end 112.25 86.75) (width 0.25) (layer "F.Cu") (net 2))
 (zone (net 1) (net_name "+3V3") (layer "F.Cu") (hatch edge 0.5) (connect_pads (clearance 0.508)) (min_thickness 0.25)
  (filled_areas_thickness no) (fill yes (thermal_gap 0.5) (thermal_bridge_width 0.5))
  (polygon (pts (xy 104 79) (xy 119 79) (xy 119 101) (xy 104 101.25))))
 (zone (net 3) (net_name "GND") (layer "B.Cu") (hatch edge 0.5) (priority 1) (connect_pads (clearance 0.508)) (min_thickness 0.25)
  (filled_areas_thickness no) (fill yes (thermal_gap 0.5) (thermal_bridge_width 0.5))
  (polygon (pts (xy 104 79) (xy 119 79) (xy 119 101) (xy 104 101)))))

